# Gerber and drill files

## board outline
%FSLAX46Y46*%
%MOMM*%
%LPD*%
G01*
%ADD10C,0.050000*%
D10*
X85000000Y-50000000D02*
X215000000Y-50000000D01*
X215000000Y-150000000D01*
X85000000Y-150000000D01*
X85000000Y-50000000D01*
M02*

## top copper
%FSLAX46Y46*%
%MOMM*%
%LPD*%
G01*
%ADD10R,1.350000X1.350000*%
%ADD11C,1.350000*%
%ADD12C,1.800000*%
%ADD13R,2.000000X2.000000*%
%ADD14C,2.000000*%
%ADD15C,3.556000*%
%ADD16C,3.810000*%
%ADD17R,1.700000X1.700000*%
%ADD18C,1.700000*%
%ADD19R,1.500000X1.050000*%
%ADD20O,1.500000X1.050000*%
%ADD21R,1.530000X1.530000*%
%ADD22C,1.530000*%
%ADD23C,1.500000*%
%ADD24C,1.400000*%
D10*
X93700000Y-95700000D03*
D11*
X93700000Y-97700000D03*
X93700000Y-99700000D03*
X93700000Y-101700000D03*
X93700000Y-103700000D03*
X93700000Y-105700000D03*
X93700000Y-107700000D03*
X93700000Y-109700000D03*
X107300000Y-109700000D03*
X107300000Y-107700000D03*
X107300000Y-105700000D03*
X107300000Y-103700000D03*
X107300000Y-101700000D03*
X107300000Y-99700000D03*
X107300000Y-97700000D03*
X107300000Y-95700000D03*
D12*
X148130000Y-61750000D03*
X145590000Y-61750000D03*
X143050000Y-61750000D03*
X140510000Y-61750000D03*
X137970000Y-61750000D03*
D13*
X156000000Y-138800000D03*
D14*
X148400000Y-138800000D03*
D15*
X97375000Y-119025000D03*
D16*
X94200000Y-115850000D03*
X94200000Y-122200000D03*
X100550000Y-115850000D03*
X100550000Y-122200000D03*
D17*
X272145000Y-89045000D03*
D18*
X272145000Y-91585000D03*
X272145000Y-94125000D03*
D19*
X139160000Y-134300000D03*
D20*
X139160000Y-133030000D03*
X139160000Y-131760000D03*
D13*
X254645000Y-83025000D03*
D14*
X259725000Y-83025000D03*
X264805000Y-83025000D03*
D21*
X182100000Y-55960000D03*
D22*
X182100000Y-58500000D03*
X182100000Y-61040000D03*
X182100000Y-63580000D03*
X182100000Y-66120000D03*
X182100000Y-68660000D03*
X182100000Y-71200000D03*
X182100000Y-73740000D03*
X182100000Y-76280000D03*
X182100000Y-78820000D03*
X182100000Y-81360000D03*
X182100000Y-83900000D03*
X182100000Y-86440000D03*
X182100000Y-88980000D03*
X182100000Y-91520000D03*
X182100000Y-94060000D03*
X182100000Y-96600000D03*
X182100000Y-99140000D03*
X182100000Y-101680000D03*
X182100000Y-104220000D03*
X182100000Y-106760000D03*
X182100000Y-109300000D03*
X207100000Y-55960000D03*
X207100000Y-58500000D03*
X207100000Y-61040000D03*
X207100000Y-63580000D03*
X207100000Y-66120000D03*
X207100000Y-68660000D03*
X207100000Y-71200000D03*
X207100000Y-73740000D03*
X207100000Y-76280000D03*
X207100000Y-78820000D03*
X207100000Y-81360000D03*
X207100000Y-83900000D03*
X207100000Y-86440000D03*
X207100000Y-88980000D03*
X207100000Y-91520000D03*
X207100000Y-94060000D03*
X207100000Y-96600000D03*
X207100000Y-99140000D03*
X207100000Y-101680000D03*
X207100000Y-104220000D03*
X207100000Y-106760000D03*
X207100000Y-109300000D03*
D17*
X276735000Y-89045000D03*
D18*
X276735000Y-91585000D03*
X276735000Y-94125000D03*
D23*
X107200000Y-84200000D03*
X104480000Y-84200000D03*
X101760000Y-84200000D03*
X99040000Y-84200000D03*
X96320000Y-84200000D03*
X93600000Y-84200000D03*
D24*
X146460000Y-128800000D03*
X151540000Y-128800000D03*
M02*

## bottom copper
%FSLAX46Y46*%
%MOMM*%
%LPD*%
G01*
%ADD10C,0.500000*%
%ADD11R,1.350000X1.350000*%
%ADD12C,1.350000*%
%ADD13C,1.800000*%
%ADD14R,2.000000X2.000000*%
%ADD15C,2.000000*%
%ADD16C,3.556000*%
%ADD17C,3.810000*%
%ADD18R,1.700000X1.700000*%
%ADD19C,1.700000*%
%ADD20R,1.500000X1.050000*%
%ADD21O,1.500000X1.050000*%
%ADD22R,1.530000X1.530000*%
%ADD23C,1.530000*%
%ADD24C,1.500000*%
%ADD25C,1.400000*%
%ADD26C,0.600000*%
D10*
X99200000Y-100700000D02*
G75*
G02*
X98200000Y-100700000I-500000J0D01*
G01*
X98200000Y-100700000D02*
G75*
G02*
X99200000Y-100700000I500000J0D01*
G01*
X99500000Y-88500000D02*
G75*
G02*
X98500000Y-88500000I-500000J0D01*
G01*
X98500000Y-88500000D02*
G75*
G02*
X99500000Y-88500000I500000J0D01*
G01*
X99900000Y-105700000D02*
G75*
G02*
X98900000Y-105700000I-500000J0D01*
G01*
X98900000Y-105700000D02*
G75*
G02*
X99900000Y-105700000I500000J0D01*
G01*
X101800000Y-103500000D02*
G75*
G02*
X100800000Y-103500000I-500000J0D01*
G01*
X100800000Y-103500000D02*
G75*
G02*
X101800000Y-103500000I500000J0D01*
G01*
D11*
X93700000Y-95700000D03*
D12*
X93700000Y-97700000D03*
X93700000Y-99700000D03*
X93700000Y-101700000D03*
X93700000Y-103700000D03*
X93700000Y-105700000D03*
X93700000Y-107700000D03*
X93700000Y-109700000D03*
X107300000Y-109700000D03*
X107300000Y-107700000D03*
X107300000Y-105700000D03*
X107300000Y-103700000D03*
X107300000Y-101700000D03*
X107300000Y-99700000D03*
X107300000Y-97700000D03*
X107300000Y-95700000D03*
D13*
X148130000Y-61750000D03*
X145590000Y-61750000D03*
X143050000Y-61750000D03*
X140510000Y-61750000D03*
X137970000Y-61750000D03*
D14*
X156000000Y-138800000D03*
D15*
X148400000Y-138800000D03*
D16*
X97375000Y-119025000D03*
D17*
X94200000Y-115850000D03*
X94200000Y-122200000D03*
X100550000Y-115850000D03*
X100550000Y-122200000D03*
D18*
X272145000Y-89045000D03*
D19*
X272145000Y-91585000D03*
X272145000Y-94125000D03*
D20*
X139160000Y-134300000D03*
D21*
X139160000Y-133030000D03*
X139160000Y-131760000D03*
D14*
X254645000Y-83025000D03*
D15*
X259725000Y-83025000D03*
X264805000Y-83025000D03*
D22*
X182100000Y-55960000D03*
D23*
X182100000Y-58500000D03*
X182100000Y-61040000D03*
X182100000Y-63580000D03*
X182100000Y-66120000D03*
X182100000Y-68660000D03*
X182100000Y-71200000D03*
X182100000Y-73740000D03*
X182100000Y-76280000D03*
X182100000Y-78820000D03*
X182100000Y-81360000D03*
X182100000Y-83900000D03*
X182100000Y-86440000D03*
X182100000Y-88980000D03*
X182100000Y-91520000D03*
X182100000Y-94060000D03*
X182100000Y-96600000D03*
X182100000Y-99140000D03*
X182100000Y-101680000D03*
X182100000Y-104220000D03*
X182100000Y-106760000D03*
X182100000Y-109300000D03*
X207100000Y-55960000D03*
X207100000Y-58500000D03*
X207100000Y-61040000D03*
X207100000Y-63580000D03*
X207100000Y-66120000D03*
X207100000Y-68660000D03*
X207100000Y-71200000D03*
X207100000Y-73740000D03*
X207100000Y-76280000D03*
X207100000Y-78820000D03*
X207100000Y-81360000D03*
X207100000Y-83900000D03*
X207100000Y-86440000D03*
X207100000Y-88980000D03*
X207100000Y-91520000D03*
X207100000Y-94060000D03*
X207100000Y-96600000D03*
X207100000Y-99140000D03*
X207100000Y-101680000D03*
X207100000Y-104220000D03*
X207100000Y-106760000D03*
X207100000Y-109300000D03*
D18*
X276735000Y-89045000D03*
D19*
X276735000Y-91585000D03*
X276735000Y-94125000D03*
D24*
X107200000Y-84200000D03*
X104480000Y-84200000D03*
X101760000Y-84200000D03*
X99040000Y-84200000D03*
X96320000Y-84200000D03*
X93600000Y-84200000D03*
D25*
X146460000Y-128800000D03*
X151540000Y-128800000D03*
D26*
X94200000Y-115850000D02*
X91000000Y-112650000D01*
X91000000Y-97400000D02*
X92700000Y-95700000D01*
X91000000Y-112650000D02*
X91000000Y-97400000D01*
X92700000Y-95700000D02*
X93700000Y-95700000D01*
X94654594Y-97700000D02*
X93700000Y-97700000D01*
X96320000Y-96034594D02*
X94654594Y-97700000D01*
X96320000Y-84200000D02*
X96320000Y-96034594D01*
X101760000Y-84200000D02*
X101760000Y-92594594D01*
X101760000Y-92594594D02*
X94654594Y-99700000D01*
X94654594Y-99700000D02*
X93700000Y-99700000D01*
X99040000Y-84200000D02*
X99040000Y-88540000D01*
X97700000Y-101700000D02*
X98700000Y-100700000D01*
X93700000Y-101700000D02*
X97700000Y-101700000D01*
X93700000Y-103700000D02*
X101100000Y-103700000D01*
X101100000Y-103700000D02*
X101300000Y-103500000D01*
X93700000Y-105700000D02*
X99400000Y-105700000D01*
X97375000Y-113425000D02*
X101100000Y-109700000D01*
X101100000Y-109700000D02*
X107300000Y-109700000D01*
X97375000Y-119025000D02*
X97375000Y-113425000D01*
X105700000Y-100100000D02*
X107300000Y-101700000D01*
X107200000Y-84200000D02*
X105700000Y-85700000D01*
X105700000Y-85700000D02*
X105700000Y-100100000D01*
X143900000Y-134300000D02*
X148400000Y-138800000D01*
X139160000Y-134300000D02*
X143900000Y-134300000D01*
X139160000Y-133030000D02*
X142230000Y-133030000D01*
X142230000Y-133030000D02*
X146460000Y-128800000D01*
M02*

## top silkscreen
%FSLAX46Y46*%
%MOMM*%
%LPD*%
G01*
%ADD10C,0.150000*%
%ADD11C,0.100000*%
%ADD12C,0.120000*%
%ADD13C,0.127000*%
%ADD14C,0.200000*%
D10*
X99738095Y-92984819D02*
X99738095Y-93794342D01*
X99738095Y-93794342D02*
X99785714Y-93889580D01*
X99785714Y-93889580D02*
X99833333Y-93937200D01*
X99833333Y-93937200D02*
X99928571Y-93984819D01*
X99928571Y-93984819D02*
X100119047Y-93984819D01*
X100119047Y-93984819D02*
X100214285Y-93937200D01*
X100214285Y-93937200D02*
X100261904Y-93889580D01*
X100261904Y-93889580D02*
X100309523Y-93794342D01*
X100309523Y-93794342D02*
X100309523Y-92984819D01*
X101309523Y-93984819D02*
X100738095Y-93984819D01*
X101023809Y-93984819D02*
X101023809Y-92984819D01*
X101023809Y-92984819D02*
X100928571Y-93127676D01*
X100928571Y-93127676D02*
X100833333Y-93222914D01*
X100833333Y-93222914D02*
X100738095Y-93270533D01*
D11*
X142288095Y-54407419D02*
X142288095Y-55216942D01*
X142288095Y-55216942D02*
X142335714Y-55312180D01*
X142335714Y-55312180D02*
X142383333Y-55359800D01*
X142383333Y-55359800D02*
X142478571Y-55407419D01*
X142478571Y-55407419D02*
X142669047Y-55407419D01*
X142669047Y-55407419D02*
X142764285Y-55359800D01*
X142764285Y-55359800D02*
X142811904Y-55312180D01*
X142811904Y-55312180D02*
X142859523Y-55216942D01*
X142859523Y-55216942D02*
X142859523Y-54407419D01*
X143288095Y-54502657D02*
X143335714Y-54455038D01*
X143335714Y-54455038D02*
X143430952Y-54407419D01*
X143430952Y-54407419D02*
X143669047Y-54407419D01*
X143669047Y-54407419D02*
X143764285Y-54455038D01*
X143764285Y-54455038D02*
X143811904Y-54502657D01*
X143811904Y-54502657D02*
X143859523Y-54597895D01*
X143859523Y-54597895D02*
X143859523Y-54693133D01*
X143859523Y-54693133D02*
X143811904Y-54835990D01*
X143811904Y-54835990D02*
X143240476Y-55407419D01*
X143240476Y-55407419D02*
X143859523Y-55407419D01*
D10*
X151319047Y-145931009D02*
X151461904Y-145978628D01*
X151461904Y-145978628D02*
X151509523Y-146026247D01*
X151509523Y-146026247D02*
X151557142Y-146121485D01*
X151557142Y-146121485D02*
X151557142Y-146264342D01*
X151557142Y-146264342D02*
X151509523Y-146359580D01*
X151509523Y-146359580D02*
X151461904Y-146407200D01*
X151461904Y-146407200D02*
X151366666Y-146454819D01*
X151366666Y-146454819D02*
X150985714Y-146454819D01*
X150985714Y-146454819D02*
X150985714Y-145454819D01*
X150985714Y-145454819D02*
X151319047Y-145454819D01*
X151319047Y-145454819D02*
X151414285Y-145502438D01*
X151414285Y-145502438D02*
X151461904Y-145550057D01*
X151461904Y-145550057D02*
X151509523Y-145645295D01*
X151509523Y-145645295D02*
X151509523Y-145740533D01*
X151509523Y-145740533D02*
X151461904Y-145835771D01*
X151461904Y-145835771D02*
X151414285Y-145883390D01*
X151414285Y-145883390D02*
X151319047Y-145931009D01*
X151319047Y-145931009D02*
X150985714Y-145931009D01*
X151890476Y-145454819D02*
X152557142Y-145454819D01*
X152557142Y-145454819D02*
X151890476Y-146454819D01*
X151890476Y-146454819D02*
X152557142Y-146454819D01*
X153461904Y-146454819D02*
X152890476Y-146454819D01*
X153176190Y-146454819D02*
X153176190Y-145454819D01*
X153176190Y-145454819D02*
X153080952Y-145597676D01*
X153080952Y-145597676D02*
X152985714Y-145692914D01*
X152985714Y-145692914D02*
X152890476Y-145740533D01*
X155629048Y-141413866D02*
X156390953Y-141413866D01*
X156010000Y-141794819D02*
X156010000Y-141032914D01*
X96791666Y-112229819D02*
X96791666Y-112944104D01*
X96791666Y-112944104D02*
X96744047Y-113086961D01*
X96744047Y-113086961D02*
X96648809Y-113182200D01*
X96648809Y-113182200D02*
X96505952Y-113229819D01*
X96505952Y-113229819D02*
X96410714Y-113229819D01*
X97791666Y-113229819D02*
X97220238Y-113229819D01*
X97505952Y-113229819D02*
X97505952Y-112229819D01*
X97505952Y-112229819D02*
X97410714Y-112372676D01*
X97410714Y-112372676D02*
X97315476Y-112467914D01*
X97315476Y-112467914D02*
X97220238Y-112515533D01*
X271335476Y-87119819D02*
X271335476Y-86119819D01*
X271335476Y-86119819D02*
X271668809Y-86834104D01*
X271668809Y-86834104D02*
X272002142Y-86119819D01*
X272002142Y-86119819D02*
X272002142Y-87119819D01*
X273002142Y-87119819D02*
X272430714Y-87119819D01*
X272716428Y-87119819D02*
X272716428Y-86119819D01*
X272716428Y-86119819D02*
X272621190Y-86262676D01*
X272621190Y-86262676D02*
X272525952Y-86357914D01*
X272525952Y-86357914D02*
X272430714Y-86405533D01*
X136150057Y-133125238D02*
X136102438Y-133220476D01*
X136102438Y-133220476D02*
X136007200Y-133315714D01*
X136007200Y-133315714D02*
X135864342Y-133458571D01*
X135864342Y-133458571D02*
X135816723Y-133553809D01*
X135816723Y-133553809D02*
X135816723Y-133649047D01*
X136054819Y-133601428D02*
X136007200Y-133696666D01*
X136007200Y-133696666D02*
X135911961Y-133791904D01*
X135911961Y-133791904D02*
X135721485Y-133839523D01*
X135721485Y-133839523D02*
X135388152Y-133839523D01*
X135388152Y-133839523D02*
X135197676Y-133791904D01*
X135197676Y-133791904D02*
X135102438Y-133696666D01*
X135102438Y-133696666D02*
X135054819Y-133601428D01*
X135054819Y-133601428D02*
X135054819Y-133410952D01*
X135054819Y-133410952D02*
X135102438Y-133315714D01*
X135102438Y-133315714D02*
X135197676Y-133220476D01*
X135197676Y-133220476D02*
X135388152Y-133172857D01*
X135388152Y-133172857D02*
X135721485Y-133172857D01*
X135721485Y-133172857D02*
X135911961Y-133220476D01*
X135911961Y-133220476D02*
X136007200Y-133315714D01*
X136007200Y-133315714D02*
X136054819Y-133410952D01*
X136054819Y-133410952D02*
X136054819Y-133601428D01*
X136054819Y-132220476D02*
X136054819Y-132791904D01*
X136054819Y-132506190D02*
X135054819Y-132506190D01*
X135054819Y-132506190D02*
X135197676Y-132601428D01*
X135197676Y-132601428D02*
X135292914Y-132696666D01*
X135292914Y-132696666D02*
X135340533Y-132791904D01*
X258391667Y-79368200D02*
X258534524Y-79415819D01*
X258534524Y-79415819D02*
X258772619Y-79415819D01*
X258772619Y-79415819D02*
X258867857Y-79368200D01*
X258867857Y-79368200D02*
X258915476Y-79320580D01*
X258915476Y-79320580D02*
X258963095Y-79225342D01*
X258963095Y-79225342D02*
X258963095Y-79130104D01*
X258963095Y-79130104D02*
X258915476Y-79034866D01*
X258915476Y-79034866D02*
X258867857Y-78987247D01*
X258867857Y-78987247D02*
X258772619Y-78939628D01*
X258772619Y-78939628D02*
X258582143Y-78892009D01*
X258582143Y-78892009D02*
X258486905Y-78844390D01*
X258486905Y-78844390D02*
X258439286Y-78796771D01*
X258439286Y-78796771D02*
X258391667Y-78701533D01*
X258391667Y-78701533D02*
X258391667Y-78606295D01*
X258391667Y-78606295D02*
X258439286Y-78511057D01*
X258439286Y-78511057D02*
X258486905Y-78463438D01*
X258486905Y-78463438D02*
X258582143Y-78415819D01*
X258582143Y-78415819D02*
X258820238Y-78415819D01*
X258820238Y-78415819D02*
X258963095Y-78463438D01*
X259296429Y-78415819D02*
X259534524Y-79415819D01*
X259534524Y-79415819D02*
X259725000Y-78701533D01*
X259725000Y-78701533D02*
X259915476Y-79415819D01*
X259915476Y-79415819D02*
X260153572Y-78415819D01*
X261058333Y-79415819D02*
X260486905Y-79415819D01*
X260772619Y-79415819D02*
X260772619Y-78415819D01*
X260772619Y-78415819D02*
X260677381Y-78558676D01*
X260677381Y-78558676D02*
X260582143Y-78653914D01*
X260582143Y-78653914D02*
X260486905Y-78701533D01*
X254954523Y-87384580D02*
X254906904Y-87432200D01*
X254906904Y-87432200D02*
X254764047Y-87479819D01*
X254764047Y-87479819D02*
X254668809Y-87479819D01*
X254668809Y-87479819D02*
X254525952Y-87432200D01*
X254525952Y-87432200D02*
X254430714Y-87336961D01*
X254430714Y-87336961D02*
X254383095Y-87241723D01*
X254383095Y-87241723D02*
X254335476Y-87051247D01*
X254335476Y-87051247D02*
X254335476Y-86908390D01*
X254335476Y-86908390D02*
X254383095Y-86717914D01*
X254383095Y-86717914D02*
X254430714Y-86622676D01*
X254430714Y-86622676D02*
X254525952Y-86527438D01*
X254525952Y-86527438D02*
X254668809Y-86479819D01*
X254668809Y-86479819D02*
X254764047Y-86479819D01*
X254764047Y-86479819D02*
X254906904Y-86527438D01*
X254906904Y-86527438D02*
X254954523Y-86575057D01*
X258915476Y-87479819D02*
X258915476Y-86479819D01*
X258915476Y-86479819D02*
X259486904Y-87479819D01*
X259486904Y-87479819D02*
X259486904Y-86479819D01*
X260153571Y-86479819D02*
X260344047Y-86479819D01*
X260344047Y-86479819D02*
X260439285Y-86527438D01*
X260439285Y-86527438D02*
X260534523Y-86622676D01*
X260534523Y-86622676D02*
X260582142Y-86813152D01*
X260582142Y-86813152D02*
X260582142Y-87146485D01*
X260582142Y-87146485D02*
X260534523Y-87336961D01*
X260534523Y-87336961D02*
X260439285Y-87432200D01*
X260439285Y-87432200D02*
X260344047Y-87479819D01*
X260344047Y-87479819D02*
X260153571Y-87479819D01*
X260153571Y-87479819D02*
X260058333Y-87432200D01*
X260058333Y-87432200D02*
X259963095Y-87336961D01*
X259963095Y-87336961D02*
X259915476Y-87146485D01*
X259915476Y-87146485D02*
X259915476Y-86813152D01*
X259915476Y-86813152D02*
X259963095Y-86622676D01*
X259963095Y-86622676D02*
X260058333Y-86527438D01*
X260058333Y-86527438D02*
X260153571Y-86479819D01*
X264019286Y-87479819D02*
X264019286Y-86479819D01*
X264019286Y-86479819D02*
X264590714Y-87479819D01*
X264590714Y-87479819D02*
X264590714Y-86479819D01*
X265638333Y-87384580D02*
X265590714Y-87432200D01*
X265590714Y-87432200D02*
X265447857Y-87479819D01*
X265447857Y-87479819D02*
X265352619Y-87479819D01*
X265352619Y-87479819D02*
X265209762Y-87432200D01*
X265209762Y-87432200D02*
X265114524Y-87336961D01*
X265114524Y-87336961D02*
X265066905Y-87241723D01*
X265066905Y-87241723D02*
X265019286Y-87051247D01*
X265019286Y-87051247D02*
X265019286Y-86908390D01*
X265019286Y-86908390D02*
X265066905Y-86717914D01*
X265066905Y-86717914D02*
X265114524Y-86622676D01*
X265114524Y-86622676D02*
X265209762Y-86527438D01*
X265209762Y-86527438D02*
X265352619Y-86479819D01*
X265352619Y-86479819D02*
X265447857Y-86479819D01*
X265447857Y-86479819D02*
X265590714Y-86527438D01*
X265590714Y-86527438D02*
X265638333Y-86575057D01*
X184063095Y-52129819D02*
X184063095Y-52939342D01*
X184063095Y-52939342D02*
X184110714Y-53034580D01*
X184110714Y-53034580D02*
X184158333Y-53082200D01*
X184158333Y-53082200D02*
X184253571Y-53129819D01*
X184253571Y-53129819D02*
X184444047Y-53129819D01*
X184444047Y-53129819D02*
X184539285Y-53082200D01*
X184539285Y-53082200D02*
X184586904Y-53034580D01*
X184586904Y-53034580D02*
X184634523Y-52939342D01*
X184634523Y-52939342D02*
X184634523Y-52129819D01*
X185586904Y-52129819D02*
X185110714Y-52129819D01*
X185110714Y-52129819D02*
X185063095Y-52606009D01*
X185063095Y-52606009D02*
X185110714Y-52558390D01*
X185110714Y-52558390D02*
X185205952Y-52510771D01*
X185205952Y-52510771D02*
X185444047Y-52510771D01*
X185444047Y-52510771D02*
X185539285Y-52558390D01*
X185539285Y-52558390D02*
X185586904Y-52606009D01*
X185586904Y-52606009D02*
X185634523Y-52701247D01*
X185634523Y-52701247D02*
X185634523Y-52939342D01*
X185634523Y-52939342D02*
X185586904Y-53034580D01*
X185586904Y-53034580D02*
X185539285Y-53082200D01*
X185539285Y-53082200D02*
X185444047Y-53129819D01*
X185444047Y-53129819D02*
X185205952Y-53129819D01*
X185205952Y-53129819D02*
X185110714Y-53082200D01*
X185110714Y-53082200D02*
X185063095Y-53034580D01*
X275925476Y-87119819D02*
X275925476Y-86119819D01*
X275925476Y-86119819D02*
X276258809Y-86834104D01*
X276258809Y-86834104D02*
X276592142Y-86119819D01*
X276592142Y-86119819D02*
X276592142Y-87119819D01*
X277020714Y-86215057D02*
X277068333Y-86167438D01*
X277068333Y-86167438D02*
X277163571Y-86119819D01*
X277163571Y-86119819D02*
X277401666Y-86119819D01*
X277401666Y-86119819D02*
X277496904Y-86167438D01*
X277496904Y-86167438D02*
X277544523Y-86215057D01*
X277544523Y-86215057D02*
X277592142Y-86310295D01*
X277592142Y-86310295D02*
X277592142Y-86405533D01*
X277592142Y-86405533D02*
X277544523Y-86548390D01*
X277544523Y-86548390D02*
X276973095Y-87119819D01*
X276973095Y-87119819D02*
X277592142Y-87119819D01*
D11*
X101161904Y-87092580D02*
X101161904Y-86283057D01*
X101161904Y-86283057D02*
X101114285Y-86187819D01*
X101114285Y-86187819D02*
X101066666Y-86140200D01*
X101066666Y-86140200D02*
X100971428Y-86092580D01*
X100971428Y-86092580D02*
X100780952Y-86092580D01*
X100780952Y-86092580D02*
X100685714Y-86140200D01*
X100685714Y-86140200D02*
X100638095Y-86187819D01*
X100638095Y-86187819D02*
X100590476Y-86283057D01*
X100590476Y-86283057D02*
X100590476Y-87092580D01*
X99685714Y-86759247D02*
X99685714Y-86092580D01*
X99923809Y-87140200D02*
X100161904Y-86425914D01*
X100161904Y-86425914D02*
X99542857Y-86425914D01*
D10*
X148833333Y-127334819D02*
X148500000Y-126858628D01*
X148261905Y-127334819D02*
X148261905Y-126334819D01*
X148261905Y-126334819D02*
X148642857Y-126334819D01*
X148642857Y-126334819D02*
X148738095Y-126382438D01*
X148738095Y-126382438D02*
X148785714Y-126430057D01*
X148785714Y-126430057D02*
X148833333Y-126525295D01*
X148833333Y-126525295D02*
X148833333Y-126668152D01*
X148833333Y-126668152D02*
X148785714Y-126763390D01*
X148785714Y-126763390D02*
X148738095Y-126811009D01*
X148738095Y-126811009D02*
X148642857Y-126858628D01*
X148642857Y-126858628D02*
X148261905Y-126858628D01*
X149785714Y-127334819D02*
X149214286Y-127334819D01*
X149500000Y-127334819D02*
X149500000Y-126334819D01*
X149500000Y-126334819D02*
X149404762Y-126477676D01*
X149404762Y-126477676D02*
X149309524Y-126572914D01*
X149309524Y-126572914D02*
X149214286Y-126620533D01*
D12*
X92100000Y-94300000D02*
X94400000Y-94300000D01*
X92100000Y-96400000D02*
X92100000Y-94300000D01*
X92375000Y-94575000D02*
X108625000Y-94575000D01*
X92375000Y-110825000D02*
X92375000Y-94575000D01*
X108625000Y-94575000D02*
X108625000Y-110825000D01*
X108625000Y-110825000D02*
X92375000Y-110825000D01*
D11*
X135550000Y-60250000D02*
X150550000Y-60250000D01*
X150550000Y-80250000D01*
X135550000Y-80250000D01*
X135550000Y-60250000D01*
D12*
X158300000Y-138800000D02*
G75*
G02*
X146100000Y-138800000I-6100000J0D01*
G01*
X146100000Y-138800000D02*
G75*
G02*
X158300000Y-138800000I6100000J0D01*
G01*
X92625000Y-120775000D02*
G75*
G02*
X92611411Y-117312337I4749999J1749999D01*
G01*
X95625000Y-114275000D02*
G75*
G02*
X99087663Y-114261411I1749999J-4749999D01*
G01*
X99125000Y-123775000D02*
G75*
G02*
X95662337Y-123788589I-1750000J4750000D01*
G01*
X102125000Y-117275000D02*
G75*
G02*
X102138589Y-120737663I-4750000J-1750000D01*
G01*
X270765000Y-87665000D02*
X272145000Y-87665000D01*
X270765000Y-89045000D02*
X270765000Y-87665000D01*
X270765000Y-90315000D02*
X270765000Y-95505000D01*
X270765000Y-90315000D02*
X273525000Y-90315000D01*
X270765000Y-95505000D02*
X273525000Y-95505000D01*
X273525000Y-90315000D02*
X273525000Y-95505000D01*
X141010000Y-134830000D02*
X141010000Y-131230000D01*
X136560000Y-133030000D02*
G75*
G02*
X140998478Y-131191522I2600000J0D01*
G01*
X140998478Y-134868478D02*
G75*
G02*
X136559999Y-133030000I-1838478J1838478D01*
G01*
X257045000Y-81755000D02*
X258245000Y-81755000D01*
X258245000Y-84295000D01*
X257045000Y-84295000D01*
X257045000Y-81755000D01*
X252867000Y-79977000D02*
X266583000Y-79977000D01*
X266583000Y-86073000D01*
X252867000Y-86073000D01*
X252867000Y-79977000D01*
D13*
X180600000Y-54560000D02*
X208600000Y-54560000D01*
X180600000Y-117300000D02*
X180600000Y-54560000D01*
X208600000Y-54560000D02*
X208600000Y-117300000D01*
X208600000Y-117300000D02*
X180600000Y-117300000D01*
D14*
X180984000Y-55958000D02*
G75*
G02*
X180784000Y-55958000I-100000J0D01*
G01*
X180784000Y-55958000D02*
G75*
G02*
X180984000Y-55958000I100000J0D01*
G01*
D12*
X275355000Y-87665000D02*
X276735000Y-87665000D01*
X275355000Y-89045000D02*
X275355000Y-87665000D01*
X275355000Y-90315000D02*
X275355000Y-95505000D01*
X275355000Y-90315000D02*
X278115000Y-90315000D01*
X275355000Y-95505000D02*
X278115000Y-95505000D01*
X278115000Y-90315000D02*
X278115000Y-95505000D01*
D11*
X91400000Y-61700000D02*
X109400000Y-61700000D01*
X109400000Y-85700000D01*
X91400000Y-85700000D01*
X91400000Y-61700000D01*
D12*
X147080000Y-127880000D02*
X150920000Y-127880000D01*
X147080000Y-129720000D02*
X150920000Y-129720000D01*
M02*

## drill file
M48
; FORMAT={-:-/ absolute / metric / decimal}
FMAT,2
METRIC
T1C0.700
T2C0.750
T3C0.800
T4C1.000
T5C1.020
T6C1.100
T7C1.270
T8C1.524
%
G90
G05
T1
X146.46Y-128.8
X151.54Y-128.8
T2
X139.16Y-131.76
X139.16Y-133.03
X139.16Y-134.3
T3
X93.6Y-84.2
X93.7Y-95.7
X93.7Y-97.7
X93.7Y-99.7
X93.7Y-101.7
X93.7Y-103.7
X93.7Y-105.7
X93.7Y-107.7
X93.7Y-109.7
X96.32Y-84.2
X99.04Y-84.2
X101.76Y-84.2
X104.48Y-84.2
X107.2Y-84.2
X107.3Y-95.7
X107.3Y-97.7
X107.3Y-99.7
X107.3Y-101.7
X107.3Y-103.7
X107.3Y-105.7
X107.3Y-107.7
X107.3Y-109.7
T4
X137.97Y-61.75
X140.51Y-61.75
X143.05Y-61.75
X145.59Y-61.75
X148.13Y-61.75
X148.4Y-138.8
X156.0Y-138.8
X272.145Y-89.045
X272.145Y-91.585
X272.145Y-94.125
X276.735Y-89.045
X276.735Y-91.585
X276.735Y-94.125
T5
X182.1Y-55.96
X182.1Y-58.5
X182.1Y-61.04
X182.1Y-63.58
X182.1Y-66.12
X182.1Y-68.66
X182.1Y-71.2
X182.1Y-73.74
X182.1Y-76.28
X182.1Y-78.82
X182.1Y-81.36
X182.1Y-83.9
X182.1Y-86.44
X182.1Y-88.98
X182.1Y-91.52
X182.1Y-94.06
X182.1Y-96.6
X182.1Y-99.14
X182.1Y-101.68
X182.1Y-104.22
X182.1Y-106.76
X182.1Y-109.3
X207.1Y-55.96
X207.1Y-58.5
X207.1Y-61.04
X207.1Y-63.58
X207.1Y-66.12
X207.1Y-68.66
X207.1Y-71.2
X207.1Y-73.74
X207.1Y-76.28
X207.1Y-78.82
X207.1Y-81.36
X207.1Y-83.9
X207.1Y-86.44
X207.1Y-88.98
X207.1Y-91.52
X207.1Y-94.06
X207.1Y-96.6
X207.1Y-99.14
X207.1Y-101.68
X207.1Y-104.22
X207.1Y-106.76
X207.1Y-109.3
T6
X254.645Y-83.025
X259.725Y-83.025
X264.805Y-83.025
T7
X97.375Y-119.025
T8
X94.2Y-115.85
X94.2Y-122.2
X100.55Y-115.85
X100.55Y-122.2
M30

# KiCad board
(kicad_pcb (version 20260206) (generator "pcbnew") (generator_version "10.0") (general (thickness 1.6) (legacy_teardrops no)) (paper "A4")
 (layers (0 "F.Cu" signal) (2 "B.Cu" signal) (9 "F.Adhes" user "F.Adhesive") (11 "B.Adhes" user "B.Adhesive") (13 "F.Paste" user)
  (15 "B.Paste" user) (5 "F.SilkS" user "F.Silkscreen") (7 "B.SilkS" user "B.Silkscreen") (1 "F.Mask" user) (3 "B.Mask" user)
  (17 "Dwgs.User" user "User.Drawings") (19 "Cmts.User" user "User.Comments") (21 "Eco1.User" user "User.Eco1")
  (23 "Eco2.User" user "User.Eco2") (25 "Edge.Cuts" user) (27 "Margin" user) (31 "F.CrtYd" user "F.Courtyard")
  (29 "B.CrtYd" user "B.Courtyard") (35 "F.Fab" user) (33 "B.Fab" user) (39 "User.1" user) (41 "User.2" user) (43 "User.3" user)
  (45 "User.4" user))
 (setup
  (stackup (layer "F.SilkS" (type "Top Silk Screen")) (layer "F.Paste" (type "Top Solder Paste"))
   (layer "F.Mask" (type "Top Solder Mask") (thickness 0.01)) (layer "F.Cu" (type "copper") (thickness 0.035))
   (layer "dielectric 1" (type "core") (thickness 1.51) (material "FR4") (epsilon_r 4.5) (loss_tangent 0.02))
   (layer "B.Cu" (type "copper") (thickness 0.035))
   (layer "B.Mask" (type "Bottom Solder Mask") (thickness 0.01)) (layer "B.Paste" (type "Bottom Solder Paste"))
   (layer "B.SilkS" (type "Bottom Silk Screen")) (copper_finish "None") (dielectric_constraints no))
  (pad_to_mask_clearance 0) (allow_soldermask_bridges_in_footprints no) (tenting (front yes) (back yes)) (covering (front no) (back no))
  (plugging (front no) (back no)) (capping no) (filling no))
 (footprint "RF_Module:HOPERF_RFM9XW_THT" (layer "F.Cu") (at 93.7 95.7)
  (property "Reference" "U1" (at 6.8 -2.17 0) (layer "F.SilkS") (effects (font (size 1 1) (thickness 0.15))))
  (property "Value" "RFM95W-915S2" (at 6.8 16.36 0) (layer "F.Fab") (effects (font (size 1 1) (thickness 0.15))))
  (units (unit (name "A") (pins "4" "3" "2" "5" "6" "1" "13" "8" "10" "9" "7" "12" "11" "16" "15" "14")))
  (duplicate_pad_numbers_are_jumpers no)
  (fp_line (start -1.6 -1.4) (end 0.7 -1.4) (stroke (width 0.12) (type solid)) (layer "F.SilkS"))
  (fp_line (start -1.6 0.7) (end -1.6 -1.4) (stroke (width 0.12) (type solid)) (layer "F.SilkS"))
  (fp_line (start -1.325 -1.125) (end 14.925 -1.125) (stroke (width 0.12) (type solid)) (layer "F.SilkS"))
  (fp_line (start -1.325 15.125) (end -1.325 -1.125) (stroke (width 0.12) (type solid)) (layer "F.SilkS"))
  (fp_line (start 14.925 -1.125) (end 14.925 15.125) (stroke (width 0.12) (type solid)) (layer "F.SilkS"))
  (fp_line (start 14.925 15.125) (end -1.325 15.125) (stroke (width 0.12) (type solid)) (layer "F.SilkS"))
  (pad "1" thru_hole rect (at 0 0) (size 1.35 1.35) (drill 0.8) (layers "*.Cu" "*.Mask") (remove_unused_layers no) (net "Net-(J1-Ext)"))
  (pad "2" thru_hole circle (at 0 2) (size 1.35 1.35) (drill 0.8) (layers "*.Cu" "*.Mask") (remove_unused_layers no) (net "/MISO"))
  (pad "3" thru_hole circle (at 0 4) (size 1.35 1.35) (drill 0.8) (layers "*.Cu" "*.Mask") (remove_unused_layers no) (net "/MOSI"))
  (pad "4" thru_hole circle (at 0 6) (size 1.35 1.35) (drill 0.8) (layers "*.Cu" "*.Mask") (remove_unused_layers no) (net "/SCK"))
  (pad "5" thru_hole circle (at 0 8) (size 1.35 1.35) (drill 0.8) (layers "*.Cu" "*.Mask") (remove_unused_layers no) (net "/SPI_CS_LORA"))
  (pad "6" thru_hole circle (at 0 10) (size 1.35 1.35) (drill 0.8) (layers "*.Cu" "*.Mask") (remove_unused_layers no) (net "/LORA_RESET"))
  (pad "7" thru_hole circle (at 0 12) (size 1.35 1.35) (drill 0.8) (layers "*.Cu" "*.Mask") (remove_unused_layers no)
   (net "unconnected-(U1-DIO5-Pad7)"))
  (pad "8" thru_hole circle (at 0 14) (size 1.35 1.35) (drill 0.8) (layers "*.Cu" "*.Mask") (remove_unused_layers no) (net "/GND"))
  (pad "9" thru_hole circle (at 13.6 14) (size 1.35 1.35) (drill 0.8) (layers "*.Cu" "*.Mask") (remove_unused_layers no) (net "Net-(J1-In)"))
  (pad "10" thru_hole circle (at 13.6 12) (size 1.35 1.35) (drill 0.8) (layers "*.Cu" "*.Mask") (remove_unused_layers no)
   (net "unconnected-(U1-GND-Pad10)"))
  (pad "11" thru_hole circle (at 13.6 10) (size 1.35 1.35) (drill 0.8) (layers "*.Cu" "*.Mask") (remove_unused_layers no)
   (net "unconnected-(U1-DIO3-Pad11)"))
  (pad "12" thru_hole circle (at 13.6 8) (size 1.35 1.35) (drill 0.8) (layers "*.Cu" "*.Mask") (remove_unused_layers no)
   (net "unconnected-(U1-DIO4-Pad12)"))
  (pad "13" thru_hole circle (at 13.6 6) (size 1.35 1.35) (drill 0.8) (layers "*.Cu" "*.Mask") (remove_unused_layers no) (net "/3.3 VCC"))
  (pad "14" thru_hole circle (at 13.6 4) (size 1.35 1.35) (drill 0.8) (layers "*.Cu" "*.Mask") (remove_unused_layers no) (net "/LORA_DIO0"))
  (pad "15" thru_hole circle (at 13.6 2) (size 1.35 1.35) (drill 0.8) (layers "*.Cu" "*.Mask") (remove_unused_layers no)
   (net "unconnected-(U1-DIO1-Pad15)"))
  (pad "16" thru_hole circle (at 13.6 0) (size 1.35 1.35) (drill 0.8) (layers "*.Cu" "*.Mask") (remove_unused_layers no)
   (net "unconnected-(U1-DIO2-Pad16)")))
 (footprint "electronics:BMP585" (layer "F.Cu") (at 143.05 60.25)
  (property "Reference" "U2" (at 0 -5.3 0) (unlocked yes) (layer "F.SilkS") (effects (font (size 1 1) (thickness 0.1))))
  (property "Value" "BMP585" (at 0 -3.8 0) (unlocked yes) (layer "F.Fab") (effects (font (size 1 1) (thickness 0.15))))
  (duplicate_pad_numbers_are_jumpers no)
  (fp_rect (start -7.5 0) (end 7.5 20) (stroke (width 0.1) (type solid)) (fill no) (layer "F.SilkS"))
  (pad "1" thru_hole circle (at 5.08 1.5) (size 1.8 1.8) (drill 1) (layers "*.Cu" "*.Mask") (remove_unused_layers no) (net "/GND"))
  (pad "2" thru_hole circle (at 2.54 1.5) (size 1.8 1.8) (drill 1) (layers "*.Cu" "*.Mask") (remove_unused_layers no) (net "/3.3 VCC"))
  (pad "3" thru_hole circle (at 0 1.5) (size 1.8 1.8) (drill 1) (layers "*.Cu" "*.Mask") (remove_unused_layers no) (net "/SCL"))
  (pad "4" thru_hole circle (at -2.54 1.5) (size 1.8 1.8) (drill 1) (layers "*.Cu" "*.Mask") (remove_unused_layers no) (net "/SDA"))
  (pad "5" thru_hole circle (at -5.08 1.5) (size 1.8 1.8) (drill 1) (layers "*.Cu" "*.Mask") (remove_unused_layers no)
   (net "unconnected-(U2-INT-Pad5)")))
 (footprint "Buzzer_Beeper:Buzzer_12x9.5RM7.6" (layer "F.Cu") (at 156 138.8 180)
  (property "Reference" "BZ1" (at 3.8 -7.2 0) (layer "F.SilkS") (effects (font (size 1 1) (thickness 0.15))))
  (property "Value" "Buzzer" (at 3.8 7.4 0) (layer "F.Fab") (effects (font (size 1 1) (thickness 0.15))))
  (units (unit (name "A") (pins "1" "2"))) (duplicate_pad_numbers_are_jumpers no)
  (fp_circle (center 3.8 0) (end 9.9 0) (stroke (width 0.12) (type solid)) (fill no) (layer "F.SilkS"))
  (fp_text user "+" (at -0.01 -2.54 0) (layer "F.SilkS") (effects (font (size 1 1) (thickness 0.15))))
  (pad "1" thru_hole rect (at 0 0 180) (size 2 2) (drill 1) (layers "*.Cu" "*.Mask") (remove_unused_layers no) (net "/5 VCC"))
  (pad "2" thru_hole circle (at 7.6 0 180) (size 2 2) (drill 1) (layers "*.Cu" "*.Mask") (remove_unused_layers no) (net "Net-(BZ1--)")))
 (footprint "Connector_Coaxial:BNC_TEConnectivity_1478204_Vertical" (layer "F.Cu") (at 97.375 119.025)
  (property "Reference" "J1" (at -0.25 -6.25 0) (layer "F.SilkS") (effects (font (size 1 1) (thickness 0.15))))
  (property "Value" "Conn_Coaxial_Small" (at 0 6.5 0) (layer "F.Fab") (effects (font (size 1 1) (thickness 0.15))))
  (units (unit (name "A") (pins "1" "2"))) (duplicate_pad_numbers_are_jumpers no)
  (fp_arc (start -4.75 1.75) (mid -5.062075 0.019867) (end -4.763589 -1.712663) (stroke (width 0.12) (type solid)) (layer "F.SilkS"))
  (fp_arc (start -1.75 -4.75) (mid -0.019867 -5.062075) (end 1.712663 -4.763589) (stroke (width 0.12) (type solid)) (layer "F.SilkS"))
  (fp_arc (start 1.75 4.75) (mid 0.019867 5.062075) (end -1.712663 4.763589) (stroke (width 0.12) (type solid)) (layer "F.SilkS"))
  (fp_arc (start 4.75 -1.75) (mid 5.062075 -0.019867) (end 4.763589 1.712663) (stroke (width 0.12) (type solid)) (layer "F.SilkS"))
  (pad "1" thru_hole circle (at 0 0) (size 3.556 3.556) (drill 1.27) (layers "*.Cu" "*.Mask") (remove_unused_layers no) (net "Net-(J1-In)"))
  (pad "2" thru_hole circle (at -3.175 -3.175) (size 3.81 3.81) (drill 1.524) (layers "*.Cu" "*.Mask") (remove_unused_layers no)
   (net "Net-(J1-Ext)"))
  (pad "2" thru_hole circle (at -3.175 3.175) (size 3.81 3.81) (drill 1.524) (layers "*.Cu" "*.Mask") (remove_unused_layers no)
   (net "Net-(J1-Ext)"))
  (pad "2" thru_hole circle (at 3.175 -3.175) (size 3.81 3.81) (drill 1.524) (layers "*.Cu" "*.Mask") (remove_unused_layers no)
   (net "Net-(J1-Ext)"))
  (pad "2" thru_hole circle (at 3.175 3.175) (size 3.81 3.81) (drill 1.524) (layers "*.Cu" "*.Mask") (remove_unused_layers no)
   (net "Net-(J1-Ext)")))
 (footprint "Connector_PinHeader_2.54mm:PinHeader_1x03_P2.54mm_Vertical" (layer "F.Cu") (at 272.145 89.045)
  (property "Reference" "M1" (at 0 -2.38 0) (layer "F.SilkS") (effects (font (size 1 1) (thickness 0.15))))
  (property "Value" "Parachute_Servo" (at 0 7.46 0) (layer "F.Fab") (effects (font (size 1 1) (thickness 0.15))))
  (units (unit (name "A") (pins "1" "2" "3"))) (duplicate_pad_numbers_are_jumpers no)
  (fp_line (start -1.38 -1.38) (end 0 -1.38) (stroke (width 0.12) (type solid)) (layer "F.SilkS"))
  (fp_line (start -1.38 0) (end -1.38 -1.38) (stroke (width 0.12) (type solid)) (layer "F.SilkS"))
  (fp_line (start -1.38 1.27) (end -1.38 6.46) (stroke (width 0.12) (type solid)) (layer "F.SilkS"))
  (fp_line (start -1.38 1.27) (end 1.38 1.27) (stroke (width 0.12) (type solid)) (layer "F.SilkS"))
  (fp_line (start -1.38 6.46) (end 1.38 6.46) (stroke (width 0.12) (type solid)) (layer "F.SilkS"))
  (fp_line (start 1.38 1.27) (end 1.38 6.46) (stroke (width 0.12) (type solid)) (layer "F.SilkS"))
  (pad "1" thru_hole rect (at 0 0) (size 1.7 1.7) (drill 1) (layers "*.Cu" "*.Mask") (remove_unused_layers no) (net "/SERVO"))
  (pad "2" thru_hole circle (at 0 2.54) (size 1.7 1.7) (drill 1) (layers "*.Cu" "*.Mask") (remove_unused_layers no) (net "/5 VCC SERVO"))
  (pad "3" thru_hole circle (at 0 5.08) (size 1.7 1.7) (drill 1) (layers "*.Cu" "*.Mask") (remove_unused_layers no) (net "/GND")))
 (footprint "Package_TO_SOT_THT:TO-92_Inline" (layer "F.Cu") (at 139.16 134.3 90)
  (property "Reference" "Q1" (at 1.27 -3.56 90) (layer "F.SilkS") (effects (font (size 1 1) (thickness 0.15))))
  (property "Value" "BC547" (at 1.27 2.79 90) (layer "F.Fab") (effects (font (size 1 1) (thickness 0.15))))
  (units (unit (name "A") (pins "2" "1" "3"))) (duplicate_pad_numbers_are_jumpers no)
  (fp_line (start -0.53 1.85) (end 3.07 1.85) (stroke (width 0.12) (type solid)) (layer "F.SilkS"))
  (fp_arc (start 1.27 -2.6) (mid 3.672087 -0.994977) (end 3.108478 1.838478) (stroke (width 0.12) (type solid)) (layer "F.SilkS"))
  (fp_arc (start -0.568478 1.838478) (mid -1.132087 -0.994977) (end 1.27 -2.6) (stroke (width 0.12) (type solid)) (layer "F.SilkS"))
  (pad "1" thru_hole rect (at 0 0 90) (size 1.05 1.5) (drill 0.75) (layers "*.Cu" "*.Mask") (remove_unused_layers no) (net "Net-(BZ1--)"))
  (pad "2" thru_hole oval (at 1.27 0 90) (size 1.05 1.5) (drill 0.75) (layers "*.Cu" "*.Mask") (remove_unused_layers no) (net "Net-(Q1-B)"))
  (pad "3" thru_hole oval (at 2.54 0 90) (size 1.05 1.5) (drill 0.75) (layers "*.Cu" "*.Mask") (remove_unused_layers no) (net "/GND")))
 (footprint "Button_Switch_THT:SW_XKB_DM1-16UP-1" (layer "F.Cu") (at 254.645 83.025)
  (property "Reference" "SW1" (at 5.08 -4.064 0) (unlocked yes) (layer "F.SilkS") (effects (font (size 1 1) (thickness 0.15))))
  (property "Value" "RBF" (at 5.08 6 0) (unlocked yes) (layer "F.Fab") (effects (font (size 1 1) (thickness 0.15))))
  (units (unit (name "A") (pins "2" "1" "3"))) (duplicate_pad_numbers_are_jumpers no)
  (fp_rect (start 2.4 -1.27) (end 3.6 1.27) (stroke (width 0.12) (type solid)) (fill no) (layer "F.SilkS"))
  (fp_rect (start 11.938 -3.048) (end -1.778 3.048) (stroke (width 0.12) (type solid)) (fill no) (layer "F.SilkS"))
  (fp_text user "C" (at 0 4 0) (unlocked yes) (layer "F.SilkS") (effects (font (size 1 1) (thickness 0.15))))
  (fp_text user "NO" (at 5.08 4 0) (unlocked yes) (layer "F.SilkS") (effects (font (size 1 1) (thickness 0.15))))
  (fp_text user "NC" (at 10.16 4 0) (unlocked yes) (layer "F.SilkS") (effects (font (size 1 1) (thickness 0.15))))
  (pad "1" thru_hole rect (at 0 0) (size 2 2) (drill 1.1) (layers "*.Cu" "*.Mask") (remove_unused_layers no) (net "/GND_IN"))
  (pad "2" thru_hole circle (at 5.08 0) (size 2 2) (drill 1.1) (layers "*.Cu" "*.Mask") (remove_unused_layers no) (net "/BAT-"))
  (pad "3" thru_hole circle (at 10.16 0) (size 2 2) (drill 1.1) (layers "*.Cu" "*.Mask") (remove_unused_layers no)
   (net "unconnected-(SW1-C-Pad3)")))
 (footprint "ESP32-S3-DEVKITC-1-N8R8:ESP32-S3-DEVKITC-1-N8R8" (layer "F.Cu") (at 194.6 85.93)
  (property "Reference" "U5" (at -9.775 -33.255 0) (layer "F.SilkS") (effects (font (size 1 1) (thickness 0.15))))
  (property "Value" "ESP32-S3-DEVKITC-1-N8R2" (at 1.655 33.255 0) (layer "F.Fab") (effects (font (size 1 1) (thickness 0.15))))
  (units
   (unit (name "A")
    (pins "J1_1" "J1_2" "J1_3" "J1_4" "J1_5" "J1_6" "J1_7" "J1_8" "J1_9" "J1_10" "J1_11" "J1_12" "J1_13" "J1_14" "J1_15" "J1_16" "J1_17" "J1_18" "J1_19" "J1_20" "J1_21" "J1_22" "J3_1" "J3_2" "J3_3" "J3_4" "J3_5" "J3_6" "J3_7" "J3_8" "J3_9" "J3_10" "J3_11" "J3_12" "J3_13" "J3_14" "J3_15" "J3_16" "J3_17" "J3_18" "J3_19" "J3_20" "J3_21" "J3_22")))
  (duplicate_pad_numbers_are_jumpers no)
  (fp_line (start -14 -31.37) (end 14 -31.37) (stroke (width 0.127) (type solid)) (layer "F.SilkS"))
  (fp_line (start -14 31.37) (end -14 -31.37) (stroke (width 0.127) (type solid)) (layer "F.SilkS"))
  (fp_line (start 14 -31.37) (end 14 31.37) (stroke (width 0.127) (type solid)) (layer "F.SilkS"))
  (fp_line (start 14 31.37) (end -14 31.37) (stroke (width 0.127) (type solid)) (layer "F.SilkS"))
  (fp_circle (center -13.716 -29.972) (end -13.616 -29.972) (stroke (width 0.2) (type solid)) (fill no) (layer "F.SilkS"))
  (pad "J1_1" thru_hole rect (at -12.5 -29.97) (size 1.53 1.53) (drill 1.02) (layers "*.Cu" "*.Mask") (remove_unused_layers no)
   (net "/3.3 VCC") (solder_mask_margin 0.102))
  (pad "J1_2" thru_hole circle (at -12.5 -27.43) (size 1.53 1.53) (drill 1.02) (layers "*.Cu" "*.Mask") (remove_unused_layers no)
   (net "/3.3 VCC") (solder_mask_margin 0.102))
  (pad "J1_3" thru_hole circle (at -12.5 -24.89) (size 1.53 1.53) (drill 1.02) (layers "*.Cu" "*.Mask") (remove_unused_layers no)
   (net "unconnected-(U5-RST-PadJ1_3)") (solder_mask_margin 0.102))
  (pad "J1_4" thru_hole circle (at -12.5 -22.35) (size 1.53 1.53) (drill 1.02) (layers "*.Cu" "*.Mask") (remove_unused_layers no)
   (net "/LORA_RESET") (solder_mask_margin 0.102))
  (pad "J1_5" thru_hole circle (at -12.5 -19.81) (size 1.53 1.53) (drill 1.02) (layers "*.Cu" "*.Mask") (remove_unused_layers no)
   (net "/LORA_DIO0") (solder_mask_margin 0.102))
  (pad "J1_6" thru_hole circle (at -12.5 -17.27) (size 1.53 1.53) (drill 1.02) (layers "*.Cu" "*.Mask") (remove_unused_layers no)
   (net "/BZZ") (solder_mask_margin 0.102))
  (pad "J1_7" thru_hole circle (at -12.5 -14.73) (size 1.53 1.53) (drill 1.02) (layers "*.Cu" "*.Mask") (remove_unused_layers no)
   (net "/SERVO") (solder_mask_margin 0.102))
  (pad "J1_8" thru_hole circle (at -12.5 -12.19) (size 1.53 1.53) (drill 1.02) (layers "*.Cu" "*.Mask") (remove_unused_layers no)
   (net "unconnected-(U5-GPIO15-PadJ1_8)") (solder_mask_margin 0.102))
  (pad "J1_9" thru_hole circle (at -12.5 -9.65) (size 1.53 1.53) (drill 1.02) (layers "*.Cu" "*.Mask") (remove_unused_layers no)
   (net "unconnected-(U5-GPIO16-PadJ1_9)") (solder_mask_margin 0.102))
  (pad "J1_10" thru_hole circle (at -12.5 -7.11) (size 1.53 1.53) (drill 1.02) (layers "*.Cu" "*.Mask") (remove_unused_layers no)
   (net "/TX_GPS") (solder_mask_margin 0.102))
  (pad "J1_11" thru_hole circle (at -12.5 -4.57) (size 1.53 1.53) (drill 1.02) (layers "*.Cu" "*.Mask") (remove_unused_layers no)
   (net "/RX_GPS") (solder_mask_margin 0.102))
  (pad "J1_12" thru_hole circle (at -12.5 -2.03) (size 1.53 1.53) (drill 1.02) (layers "*.Cu" "*.Mask") (remove_unused_layers no)
   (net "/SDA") (solder_mask_margin 0.102))
  (pad "J1_13" thru_hole circle (at -12.5 0.51) (size 1.53 1.53) (drill 1.02) (layers "*.Cu" "*.Mask") (remove_unused_layers no)
   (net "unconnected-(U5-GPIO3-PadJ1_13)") (solder_mask_margin 0.102))
  (pad "J1_14" thru_hole circle (at -12.5 3.05) (size 1.53 1.53) (drill 1.02) (layers "*.Cu" "*.Mask") (remove_unused_layers no)
   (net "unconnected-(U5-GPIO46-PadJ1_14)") (solder_mask_margin 0.102))
  (pad "J1_15" thru_hole circle (at -12.5 5.59) (size 1.53 1.53) (drill 1.02) (layers "*.Cu" "*.Mask") (remove_unused_layers no)
   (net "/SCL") (solder_mask_margin 0.102))
  (pad "J1_16" thru_hole circle (at -12.5 8.13) (size 1.53 1.53) (drill 1.02) (layers "*.Cu" "*.Mask") (remove_unused_layers no)
   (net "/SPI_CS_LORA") (solder_mask_margin 0.102))
  (pad "J1_17" thru_hole circle (at -12.5 10.67) (size 1.53 1.53) (drill 1.02) (layers "*.Cu" "*.Mask") (remove_unused_layers no)
   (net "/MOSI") (solder_mask_margin 0.102))
  (pad "J1_18" thru_hole circle (at -12.5 13.21) (size 1.53 1.53) (drill 1.02) (layers "*.Cu" "*.Mask") (remove_unused_layers no)
   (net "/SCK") (solder_mask_margin 0.102))
  (pad "J1_19" thru_hole circle (at -12.5 15.75) (size 1.53 1.53) (drill 1.02) (layers "*.Cu" "*.Mask") (remove_unused_layers no)
   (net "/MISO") (solder_mask_margin 0.102))
  (pad "J1_20" thru_hole circle (at -12.5 18.29) (size 1.53 1.53) (drill 1.02) (layers "*.Cu" "*.Mask") (remove_unused_layers no)
   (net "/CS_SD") (solder_mask_margin 0.102))
  (pad "J1_21" thru_hole circle (at -12.5 20.83) (size 1.53 1.53) (drill 1.02) (layers "*.Cu" "*.Mask") (remove_unused_layers no)
   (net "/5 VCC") (solder_mask_margin 0.102))
  (pad "J1_22" thru_hole circle (at -12.5 23.37) (size 1.53 1.53) (drill 1.02) (layers "*.Cu" "*.Mask") (remove_unused_layers no)
   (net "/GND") (solder_mask_margin 0.102))
  (pad "J3_1" thru_hole circle (at 12.5 -29.97) (size 1.53 1.53) (drill 1.02) (layers "*.Cu" "*.Mask") (remove_unused_layers no)
   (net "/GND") (solder_mask_margin 0.102))
  (pad "J3_2" thru_hole circle (at 12.5 -27.43) (size 1.53 1.53) (drill 1.02) (layers "*.Cu" "*.Mask") (remove_unused_layers no)
   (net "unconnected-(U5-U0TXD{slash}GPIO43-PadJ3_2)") (solder_mask_margin 0.102))
  (pad "J3_3" thru_hole circle (at 12.5 -24.89) (size 1.53 1.53) (drill 1.02) (layers "*.Cu" "*.Mask") (remove_unused_layers no)
   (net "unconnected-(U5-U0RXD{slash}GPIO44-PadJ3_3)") (solder_mask_margin 0.102))
  (pad "J3_4" thru_hole circle (at 12.5 -22.35) (size 1.53 1.53) (drill 1.02) (layers "*.Cu" "*.Mask") (remove_unused_layers no)
   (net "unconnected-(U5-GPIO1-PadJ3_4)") (solder_mask_margin 0.102))
  (pad "J3_5" thru_hole circle (at 12.5 -19.81) (size 1.53 1.53) (drill 1.02) (layers "*.Cu" "*.Mask") (remove_unused_layers no)
   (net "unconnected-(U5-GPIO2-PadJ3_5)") (solder_mask_margin 0.102))
  (pad "J3_6" thru_hole circle (at 12.5 -17.27) (size 1.53 1.53) (drill 1.02) (layers "*.Cu" "*.Mask") (remove_unused_layers no)
   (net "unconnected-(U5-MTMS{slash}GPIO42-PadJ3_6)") (solder_mask_margin 0.102))
  (pad "J3_7" thru_hole circle (at 12.5 -14.73) (size 1.53 1.53) (drill 1.02) (layers "*.Cu" "*.Mask") (remove_unused_layers no)
   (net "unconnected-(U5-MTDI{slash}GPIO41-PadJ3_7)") (solder_mask_margin 0.102))
  (pad "J3_8" thru_hole circle (at 12.5 -12.19) (size 1.53 1.53) (drill 1.02) (layers "*.Cu" "*.Mask") (remove_unused_layers no)
   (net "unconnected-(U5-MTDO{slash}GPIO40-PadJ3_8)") (solder_mask_margin 0.102))
  (pad "J3_9" thru_hole circle (at 12.5 -9.65) (size 1.53 1.53) (drill 1.02) (layers "*.Cu" "*.Mask") (remove_unused_layers no)
   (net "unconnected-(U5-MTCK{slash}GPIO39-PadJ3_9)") (solder_mask_margin 0.102))
  (pad "J3_10" thru_hole circle (at 12.5 -7.11) (size 1.53 1.53) (drill 1.02) (layers "*.Cu" "*.Mask") (remove_unused_layers no)
   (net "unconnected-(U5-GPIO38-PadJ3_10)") (solder_mask_margin 0.102))
  (pad "J3_11" thru_hole circle (at 12.5 -4.57) (size 1.53 1.53) (drill 1.02) (layers "*.Cu" "*.Mask") (remove_unused_layers no)
   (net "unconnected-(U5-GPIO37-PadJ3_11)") (solder_mask_margin 0.102))
  (pad "J3_12" thru_hole circle (at 12.5 -2.03) (size 1.53 1.53) (drill 1.02) (layers "*.Cu" "*.Mask") (remove_unused_layers no)
   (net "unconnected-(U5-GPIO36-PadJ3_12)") (solder_mask_margin 0.102))
  (pad "J3_13" thru_hole circle (at 12.5 0.51) (size 1.53 1.53) (drill 1.02) (layers "*.Cu" "*.Mask") (remove_unused_layers no)
   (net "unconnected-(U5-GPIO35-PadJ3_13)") (solder_mask_margin 0.102))
  (pad "J3_14" thru_hole circle (at 12.5 3.05) (size 1.53 1.53) (drill 1.02) (layers "*.Cu" "*.Mask") (remove_unused_layers no)
   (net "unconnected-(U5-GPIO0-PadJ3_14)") (solder_mask_margin 0.102))
  (pad "J3_15" thru_hole circle (at 12.5 5.59) (size 1.53 1.53) (drill 1.02) (layers "*.Cu" "*.Mask") (remove_unused_layers no)
   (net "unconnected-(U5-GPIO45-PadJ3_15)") (solder_mask_margin 0.102))
  (pad "J3_16" thru_hole circle (at 12.5 8.13) (size 1.53 1.53) (drill 1.02) (layers "*.Cu" "*.Mask") (remove_unused_layers no)
   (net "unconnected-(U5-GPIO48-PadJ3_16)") (solder_mask_margin 0.102))
  (pad "J3_17" thru_hole circle (at 12.5 10.67) (size 1.53 1.53) (drill 1.02) (layers "*.Cu" "*.Mask") (remove_unused_layers no)
   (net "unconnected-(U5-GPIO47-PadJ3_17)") (solder_mask_margin 0.102))
  (pad "J3_18" thru_hole circle (at 12.5 13.21) (size 1.53 1.53) (drill 1.02) (layers "*.Cu" "*.Mask") (remove_unused_layers no)
   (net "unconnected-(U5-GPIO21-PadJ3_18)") (solder_mask_margin 0.102))
  (pad "J3_19" thru_hole circle (at 12.5 15.75) (size 1.53 1.53) (drill 1.02) (layers "*.Cu" "*.Mask") (remove_unused_layers no)
   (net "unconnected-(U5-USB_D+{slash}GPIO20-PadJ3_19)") (solder_mask_margin 0.102))
  (pad "J3_20" thru_hole circle (at 12.5 18.29) (size 1.53 1.53) (drill 1.02) (layers "*.Cu" "*.Mask") (remove_unused_layers no)
   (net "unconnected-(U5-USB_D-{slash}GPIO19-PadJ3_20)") (solder_mask_margin 0.102))
  (pad "J3_21" thru_hole circle (at 12.5 20.83) (size 1.53 1.53) (drill 1.02) (layers "*.Cu" "*.Mask") (remove_unused_layers no)
   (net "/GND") (solder_mask_margin 0.102))
  (pad "J3_22" thru_hole circle (at 12.5 23.37) (size 1.53 1.53) (drill 1.02) (layers "*.Cu" "*.Mask") (remove_unused_layers no)
   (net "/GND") (solder_mask_margin 0.102)))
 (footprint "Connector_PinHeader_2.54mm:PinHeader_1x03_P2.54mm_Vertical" (layer "F.Cu") (at 276.735 89.045)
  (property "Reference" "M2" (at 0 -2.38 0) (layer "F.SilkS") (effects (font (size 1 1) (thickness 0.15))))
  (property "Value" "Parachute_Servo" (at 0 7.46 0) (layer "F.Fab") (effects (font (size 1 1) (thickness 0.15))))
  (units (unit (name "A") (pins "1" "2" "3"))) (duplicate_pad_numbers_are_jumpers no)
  (fp_line (start -1.38 -1.38) (end 0 -1.38) (stroke (width 0.12) (type solid)) (layer "F.SilkS"))
  (fp_line (start -1.38 0) (end -1.38 -1.38) (stroke (width 0.12) (type solid)) (layer "F.SilkS"))
  (fp_line (start -1.38 1.27) (end -1.38 6.46) (stroke (width 0.12) (type solid)) (layer "F.SilkS"))
  (fp_line (start -1.38 1.27) (end 1.38 1.27) (stroke (width 0.12) (type solid)) (layer "F.SilkS"))
  (fp_line (start -1.38 6.46) (end 1.38 6.46) (stroke (width 0.12) (type solid)) (layer "F.SilkS"))
  (fp_line (start 1.38 1.27) (end 1.38 6.46) (stroke (width 0.12) (type solid)) (layer "F.SilkS"))
  (pad "1" thru_hole rect (at 0 0) (size 1.7 1.7) (drill 1) (layers "*.Cu" "*.Mask") (remove_unused_layers no) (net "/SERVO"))
  (pad "2" thru_hole circle (at 0 2.54) (size 1.7 1.7) (drill 1) (layers "*.Cu" "*.Mask") (remove_unused_layers no) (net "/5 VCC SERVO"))
  (pad "3" thru_hole circle (at 0 5.08) (size 1.7 1.7) (drill 1) (layers "*.Cu" "*.Mask") (remove_unused_layers no) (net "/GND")))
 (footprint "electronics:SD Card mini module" (layer "F.Cu") (at 100.4 85.7 180)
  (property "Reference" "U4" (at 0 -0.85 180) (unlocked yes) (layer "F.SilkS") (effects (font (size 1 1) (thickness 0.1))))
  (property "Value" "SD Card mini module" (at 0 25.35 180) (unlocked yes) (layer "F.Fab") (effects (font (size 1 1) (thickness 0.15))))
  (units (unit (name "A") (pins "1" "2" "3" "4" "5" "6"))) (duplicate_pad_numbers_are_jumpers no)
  (fp_rect (start -9 0) (end 9 24) (stroke (width 0.1) (type solid)) (fill no) (layer "F.SilkS"))
  (pad "1" thru_hole circle (at -6.8 1.5 180) (size 1.5 1.5) (drill 0.8) (layers "*.Cu" "*.Mask") (remove_unused_layers no) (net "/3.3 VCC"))
  (pad "2" thru_hole circle (at -4.08 1.5 180) (size 1.5 1.5) (drill 0.8) (layers "*.Cu" "*.Mask") (remove_unused_layers no) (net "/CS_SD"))
  (pad "3" thru_hole circle (at -1.36 1.5 180) (size 1.5 1.5) (drill 0.8) (layers "*.Cu" "*.Mask") (remove_unused_layers no) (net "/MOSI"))
  (pad "4" thru_hole circle (at 1.36 1.5 180) (size 1.5 1.5) (drill 0.8) (layers "*.Cu" "*.Mask") (remove_unused_layers no) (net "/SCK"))
  (pad "5" thru_hole circle (at 4.08 1.5 180) (size 1.5 1.5) (drill 0.8) (layers "*.Cu" "*.Mask") (remove_unused_layers no) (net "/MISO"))
  (pad "6" thru_hole circle (at 6.8 1.5 180) (size 1.5 1.5) (drill 0.8) (layers "*.Cu" "*.Mask") (remove_unused_layers no) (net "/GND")))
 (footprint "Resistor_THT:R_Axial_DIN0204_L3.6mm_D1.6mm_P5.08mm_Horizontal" (layer "F.Cu") (at 146.46 128.8)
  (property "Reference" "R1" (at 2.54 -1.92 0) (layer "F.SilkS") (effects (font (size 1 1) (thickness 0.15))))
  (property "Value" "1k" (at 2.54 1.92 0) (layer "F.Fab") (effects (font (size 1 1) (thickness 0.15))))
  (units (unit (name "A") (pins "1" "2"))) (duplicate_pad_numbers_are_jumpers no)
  (fp_line (start 0.62 -0.92) (end 4.46 -0.92) (stroke (width 0.12) (type solid)) (layer "F.SilkS"))
  (fp_line (start 0.62 0.92) (end 4.46 0.92) (stroke (width 0.12) (type solid)) (layer "F.SilkS"))
  (pad "1" thru_hole circle (at 0 0) (size 1.4 1.4) (drill 0.7) (layers "*.Cu" "*.Mask") (remove_unused_layers no) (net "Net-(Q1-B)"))
  (pad "2" thru_hole circle (at 5.08 0) (size 1.4 1.4) (drill 0.7) (layers "*.Cu" "*.Mask") (remove_unused_layers no) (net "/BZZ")))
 (gr_circle (center 98.7 100.7) (end 99.2 100.7) (stroke (width 0.5) (type solid)) (fill no) (layer "B.Cu") (net "/SCK"))
 (gr_circle (center 99 88.5) (end 98.5 88.5) (stroke (width 0.5) (type solid)) (fill no) (layer "B.Cu") (net "/SCK"))
 (gr_circle (center 99.4 105.7) (end 99.9 105.7) (stroke (width 0.5) (type solid)) (fill no) (layer "B.Cu") (net "/LORA_RESET"))
 (gr_circle (center 101.3 103.5) (end 101.8 103.5) (stroke (width 0.5) (type solid)) (fill no) (layer "B.Cu") (net "/SPI_CS_LORA"))
 (gr_rect (start 85 50) (end 215 150) (stroke (width 0.05) (type solid)) (fill no) (layer "Edge.Cuts"))
 (segment (start 94.2 115.85) (end 91 112.65) (width 0.6) (layer "B.Cu") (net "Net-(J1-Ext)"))
 (segment (start 91 97.4) (end 92.7 95.7) (width 0.6) (layer "B.Cu") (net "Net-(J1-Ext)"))
 (segment (start 91 112.65) (end 91 97.4) (width 0.6) (layer "B.Cu") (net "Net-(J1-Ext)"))
 (segment (start 92.7 95.7) (end 93.7 95.7) (width 0.6) (layer "B.Cu") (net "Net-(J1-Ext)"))
 (segment (start 94.654594 97.7) (end 93.7 97.7) (width 0.6) (layer "B.Cu") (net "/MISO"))
 (segment (start 96.32 96.034594) (end 94.654594 97.7) (width 0.6) (layer "B.Cu") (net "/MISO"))
 (segment (start 96.32 84.2) (end 96.32 96.034594) (width 0.6) (layer "B.Cu") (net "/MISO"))
 (segment (start 101.76 84.2) (end 101.76 92.594594) (width 0.6) (layer "B.Cu") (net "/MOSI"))
 (segment (start 101.76 92.594594) (end 94.654594 99.7) (width 0.6) (layer "B.Cu") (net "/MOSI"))
 (segment (start 94.654594 99.7) (end 93.7 99.7) (width 0.6) (layer "B.Cu") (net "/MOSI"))
 (segment (start 99.04 84.2) (end 99.04 88.54) (width 0.6) (layer "B.Cu") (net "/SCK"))
 (segment (start 97.7 101.7) (end 98.7 100.7) (width 0.6) (layer "B.Cu") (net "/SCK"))
 (segment (start 93.7 101.7) (end 97.7 101.7) (width 0.6) (layer "B.Cu") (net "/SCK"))
 (segment (start 93.7 103.7) (end 101.1 103.7) (width 0.6) (layer "B.Cu") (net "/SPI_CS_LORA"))
 (segment (start 101.1 103.7) (end 101.3 103.5) (width 0.6) (layer "B.Cu") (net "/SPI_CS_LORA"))
 (segment (start 93.7 105.7) (end 99.4 105.7) (width 0.6) (layer "B.Cu") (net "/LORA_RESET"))
 (segment (start 97.375 113.425) (end 101.1 109.7) (width 0.6) (layer "B.Cu") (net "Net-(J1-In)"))
 (segment (start 101.1 109.7) (end 107.3 109.7) (width 0.6) (layer "B.Cu") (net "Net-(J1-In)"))
 (segment (start 97.375 119.025) (end 97.375 113.425) (width 0.6) (layer "B.Cu") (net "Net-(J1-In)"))
 (segment (start 105.7 100.1) (end 107.3 101.7) (width 0.6) (layer "B.Cu") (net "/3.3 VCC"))
 (segment (start 107.2 84.2) (end 105.7 85.7) (width 0.6) (layer "B.Cu") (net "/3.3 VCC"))
 (segment (start 105.7 85.7) (end 105.7 100.1) (width 0.6) (layer "B.Cu") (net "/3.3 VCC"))
 (segment (start 143.9 134.3) (end 148.4 138.8) (width 0.6) (layer "B.Cu") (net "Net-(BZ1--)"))
 (segment (start 139.16 134.3) (end 143.9 134.3) (width 0.6) (layer "B.Cu") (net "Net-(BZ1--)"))
 (segment (start 139.16 133.03) (end 142.23 133.03) (width 0.6) (layer "B.Cu") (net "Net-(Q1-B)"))
 (segment (start 142.23 133.03) (end 146.46 128.8) (width 0.6) (layer "B.Cu") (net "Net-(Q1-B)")))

